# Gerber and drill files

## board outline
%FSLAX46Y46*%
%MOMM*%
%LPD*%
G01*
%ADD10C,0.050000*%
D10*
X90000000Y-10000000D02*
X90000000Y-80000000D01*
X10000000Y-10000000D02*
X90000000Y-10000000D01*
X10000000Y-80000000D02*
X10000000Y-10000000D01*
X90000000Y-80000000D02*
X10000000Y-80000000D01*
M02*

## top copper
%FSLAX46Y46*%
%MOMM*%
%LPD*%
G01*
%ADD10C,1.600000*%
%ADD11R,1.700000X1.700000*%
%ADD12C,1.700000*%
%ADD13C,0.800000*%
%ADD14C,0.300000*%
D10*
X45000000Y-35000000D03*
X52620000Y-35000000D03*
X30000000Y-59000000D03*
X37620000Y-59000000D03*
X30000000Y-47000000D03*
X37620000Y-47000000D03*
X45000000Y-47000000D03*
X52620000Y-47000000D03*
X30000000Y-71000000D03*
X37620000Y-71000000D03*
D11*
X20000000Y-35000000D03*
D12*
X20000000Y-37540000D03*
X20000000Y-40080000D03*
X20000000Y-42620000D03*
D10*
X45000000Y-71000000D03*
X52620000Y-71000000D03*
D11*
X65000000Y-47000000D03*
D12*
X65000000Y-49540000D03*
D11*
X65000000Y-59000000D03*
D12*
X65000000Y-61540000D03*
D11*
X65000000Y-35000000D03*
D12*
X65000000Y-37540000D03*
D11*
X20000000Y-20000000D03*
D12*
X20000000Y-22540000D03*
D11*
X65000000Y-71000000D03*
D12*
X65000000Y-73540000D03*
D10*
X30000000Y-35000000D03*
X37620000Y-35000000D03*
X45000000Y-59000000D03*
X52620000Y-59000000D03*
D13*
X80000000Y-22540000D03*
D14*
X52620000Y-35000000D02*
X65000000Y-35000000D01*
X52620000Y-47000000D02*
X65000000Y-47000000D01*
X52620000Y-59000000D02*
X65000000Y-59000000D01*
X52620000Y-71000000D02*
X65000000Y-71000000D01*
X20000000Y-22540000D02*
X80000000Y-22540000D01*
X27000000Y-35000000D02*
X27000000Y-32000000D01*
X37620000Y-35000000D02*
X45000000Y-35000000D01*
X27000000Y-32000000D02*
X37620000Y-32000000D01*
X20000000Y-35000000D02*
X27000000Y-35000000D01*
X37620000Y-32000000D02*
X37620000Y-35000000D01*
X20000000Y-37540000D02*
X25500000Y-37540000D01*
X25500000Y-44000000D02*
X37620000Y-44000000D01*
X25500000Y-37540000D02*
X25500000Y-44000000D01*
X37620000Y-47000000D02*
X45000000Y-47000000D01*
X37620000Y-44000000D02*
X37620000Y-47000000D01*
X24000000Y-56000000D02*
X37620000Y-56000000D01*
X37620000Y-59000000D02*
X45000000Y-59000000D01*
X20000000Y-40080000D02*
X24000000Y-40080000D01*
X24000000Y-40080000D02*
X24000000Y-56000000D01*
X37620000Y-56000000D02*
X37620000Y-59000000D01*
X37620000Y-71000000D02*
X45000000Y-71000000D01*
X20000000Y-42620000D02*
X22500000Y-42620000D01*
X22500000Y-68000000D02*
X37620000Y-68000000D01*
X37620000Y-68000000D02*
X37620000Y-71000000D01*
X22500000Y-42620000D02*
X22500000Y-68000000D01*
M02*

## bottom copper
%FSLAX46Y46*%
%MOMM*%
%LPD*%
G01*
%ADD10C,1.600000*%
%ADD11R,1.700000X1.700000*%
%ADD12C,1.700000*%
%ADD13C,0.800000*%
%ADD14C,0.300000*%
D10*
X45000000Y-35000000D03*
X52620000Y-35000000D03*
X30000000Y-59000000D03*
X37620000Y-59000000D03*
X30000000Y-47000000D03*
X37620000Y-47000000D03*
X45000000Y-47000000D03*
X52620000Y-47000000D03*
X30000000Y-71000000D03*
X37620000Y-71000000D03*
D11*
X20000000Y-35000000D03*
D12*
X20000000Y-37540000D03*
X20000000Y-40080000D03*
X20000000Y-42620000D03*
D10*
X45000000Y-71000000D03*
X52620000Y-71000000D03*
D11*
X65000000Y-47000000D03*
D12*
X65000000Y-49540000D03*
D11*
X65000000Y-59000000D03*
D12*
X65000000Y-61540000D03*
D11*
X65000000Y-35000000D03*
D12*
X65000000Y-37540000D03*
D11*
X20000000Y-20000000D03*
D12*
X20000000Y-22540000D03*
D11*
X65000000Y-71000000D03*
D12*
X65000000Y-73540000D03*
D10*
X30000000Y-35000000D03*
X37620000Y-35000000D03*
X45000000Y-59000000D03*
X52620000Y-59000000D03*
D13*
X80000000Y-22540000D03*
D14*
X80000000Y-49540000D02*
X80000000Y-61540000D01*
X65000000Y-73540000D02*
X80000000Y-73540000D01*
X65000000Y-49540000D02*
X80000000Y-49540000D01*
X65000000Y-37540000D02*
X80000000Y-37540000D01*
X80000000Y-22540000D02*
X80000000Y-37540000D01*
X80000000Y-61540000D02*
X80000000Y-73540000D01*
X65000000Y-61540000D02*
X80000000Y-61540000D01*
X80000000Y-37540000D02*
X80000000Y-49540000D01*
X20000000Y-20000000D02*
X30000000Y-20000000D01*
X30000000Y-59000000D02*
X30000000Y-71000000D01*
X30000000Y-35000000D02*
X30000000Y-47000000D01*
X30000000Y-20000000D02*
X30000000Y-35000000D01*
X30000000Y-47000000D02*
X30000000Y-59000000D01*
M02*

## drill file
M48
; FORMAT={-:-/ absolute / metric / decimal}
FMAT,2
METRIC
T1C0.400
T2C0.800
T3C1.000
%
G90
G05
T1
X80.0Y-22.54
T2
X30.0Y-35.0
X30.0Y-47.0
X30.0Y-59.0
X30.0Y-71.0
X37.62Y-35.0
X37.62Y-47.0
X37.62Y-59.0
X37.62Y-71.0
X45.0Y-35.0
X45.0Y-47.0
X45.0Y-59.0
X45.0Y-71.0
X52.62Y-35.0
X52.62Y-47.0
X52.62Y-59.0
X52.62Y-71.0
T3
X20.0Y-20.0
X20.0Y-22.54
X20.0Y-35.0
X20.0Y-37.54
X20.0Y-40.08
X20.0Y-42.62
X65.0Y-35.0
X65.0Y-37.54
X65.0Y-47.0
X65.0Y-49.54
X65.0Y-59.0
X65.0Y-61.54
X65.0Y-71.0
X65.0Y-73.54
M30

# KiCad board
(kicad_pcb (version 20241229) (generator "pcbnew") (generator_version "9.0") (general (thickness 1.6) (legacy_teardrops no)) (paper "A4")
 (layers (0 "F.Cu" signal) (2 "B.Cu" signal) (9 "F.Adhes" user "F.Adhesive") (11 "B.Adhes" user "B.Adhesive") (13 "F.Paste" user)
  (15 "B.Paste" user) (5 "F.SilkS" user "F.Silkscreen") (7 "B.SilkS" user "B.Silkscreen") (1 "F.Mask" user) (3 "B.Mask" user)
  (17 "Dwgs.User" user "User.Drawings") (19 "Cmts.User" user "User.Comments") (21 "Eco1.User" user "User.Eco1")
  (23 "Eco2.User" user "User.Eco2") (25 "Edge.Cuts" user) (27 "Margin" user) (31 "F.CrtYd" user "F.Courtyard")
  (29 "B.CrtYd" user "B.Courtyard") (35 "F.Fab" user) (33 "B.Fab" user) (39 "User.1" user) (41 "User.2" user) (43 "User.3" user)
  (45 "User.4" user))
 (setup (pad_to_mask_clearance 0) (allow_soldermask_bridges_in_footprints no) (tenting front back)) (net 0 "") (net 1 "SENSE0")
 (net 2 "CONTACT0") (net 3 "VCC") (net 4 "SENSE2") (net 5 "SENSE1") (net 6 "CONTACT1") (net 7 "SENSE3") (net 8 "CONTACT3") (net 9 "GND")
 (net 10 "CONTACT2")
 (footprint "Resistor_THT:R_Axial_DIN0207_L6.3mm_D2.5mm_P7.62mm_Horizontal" (layer "F.Cu") (at 45 35)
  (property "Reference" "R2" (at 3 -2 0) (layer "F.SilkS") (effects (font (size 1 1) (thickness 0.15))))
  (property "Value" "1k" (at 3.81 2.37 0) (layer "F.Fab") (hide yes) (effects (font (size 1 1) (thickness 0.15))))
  (pad "1" thru_hole circle (at 0 0) (size 1.6 1.6) (drill 0.8) (layers "*.Cu" "*.Mask") (remove_unused_layers no) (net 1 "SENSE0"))
  (pad "2" thru_hole circle (at 7.62 0) (size 1.6 1.6) (drill 0.8) (layers "*.Cu" "*.Mask") (remove_unused_layers no) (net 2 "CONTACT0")))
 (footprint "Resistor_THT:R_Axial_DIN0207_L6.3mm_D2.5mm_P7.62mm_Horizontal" (layer "F.Cu") (at 30 59)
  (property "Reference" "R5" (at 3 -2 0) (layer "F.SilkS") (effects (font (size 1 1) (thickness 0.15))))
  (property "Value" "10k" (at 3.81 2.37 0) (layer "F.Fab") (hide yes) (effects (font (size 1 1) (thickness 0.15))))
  (pad "1" thru_hole circle (at 0 0) (size 1.6 1.6) (drill 0.8) (layers "*.Cu" "*.Mask") (remove_unused_layers no) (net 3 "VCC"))
  (pad "2" thru_hole circle (at 7.62 0) (size 1.6 1.6) (drill 0.8) (layers "*.Cu" "*.Mask") (remove_unused_layers no) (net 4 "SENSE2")))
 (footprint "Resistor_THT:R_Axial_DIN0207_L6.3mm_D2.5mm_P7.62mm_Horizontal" (layer "F.Cu") (at 30 47)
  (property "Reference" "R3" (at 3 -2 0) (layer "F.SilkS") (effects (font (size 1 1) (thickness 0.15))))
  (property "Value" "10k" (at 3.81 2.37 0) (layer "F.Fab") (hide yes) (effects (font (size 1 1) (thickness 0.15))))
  (pad "1" thru_hole circle (at 0 0) (size 1.6 1.6) (drill 0.8) (layers "*.Cu" "*.Mask") (remove_unused_layers no) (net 3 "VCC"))
  (pad "2" thru_hole circle (at 7.62 0) (size 1.6 1.6) (drill 0.8) (layers "*.Cu" "*.Mask") (remove_unused_layers no) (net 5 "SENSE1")))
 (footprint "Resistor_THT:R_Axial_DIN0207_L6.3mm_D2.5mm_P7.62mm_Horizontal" (layer "F.Cu") (at 45 47)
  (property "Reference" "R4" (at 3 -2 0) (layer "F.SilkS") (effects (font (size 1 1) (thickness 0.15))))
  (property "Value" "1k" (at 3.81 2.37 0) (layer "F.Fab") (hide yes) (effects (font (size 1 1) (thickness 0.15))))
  (pad "1" thru_hole circle (at 0 0) (size 1.6 1.6) (drill 0.8) (layers "*.Cu" "*.Mask") (remove_unused_layers no) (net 5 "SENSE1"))
  (pad "2" thru_hole circle (at 7.62 0) (size 1.6 1.6) (drill 0.8) (layers "*.Cu" "*.Mask") (remove_unused_layers no) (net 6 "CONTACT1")))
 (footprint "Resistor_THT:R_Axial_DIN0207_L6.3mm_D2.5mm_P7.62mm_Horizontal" (layer "F.Cu") (at 30 71)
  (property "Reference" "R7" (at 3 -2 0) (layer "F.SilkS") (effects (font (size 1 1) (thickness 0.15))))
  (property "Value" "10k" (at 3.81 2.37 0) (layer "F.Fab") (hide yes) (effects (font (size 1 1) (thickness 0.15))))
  (pad "1" thru_hole circle (at 0 0) (size 1.6 1.6) (drill 0.8) (layers "*.Cu" "*.Mask") (remove_unused_layers no) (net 3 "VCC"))
  (pad "2" thru_hole circle (at 7.62 0) (size 1.6 1.6) (drill 0.8) (layers "*.Cu" "*.Mask") (remove_unused_layers no) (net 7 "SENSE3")))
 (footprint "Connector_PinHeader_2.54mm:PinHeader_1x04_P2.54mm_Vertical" (layer "F.Cu") (at 20 35)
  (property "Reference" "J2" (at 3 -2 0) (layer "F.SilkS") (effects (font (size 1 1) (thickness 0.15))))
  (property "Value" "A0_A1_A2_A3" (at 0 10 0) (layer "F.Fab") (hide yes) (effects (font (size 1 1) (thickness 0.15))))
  (pad "1" thru_hole rect (at 0 0) (size 1.7 1.7) (drill 1) (layers "*.Cu" "*.Mask") (remove_unused_layers no) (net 1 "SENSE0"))
  (pad "2" thru_hole circle (at 0 2.54) (size 1.7 1.7) (drill 1) (layers "*.Cu" "*.Mask") (remove_unused_layers no) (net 5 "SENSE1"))
  (pad "3" thru_hole circle (at 0 5.08) (size 1.7 1.7) (drill 1) (layers "*.Cu" "*.Mask") (remove_unused_layers no) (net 4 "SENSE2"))
  (pad "4" thru_hole circle (at 0 7.62) (size 1.7 1.7) (drill 1) (layers "*.Cu" "*.Mask") (remove_unused_layers no) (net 7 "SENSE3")))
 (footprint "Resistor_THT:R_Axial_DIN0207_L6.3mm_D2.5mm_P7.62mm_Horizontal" (layer "F.Cu") (at 45 71)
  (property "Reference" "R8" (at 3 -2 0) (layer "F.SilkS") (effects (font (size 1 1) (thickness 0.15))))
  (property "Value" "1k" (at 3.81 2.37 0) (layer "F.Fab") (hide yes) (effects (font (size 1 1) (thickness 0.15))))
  (pad "1" thru_hole circle (at 0 0) (size 1.6 1.6) (drill 0.8) (layers "*.Cu" "*.Mask") (remove_unused_layers no) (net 7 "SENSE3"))
  (pad "2" thru_hole circle (at 7.62 0) (size 1.6 1.6) (drill 0.8) (layers "*.Cu" "*.Mask") (remove_unused_layers no) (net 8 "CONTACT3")))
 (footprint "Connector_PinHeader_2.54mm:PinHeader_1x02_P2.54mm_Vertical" (layer "F.Cu") (at 65 47)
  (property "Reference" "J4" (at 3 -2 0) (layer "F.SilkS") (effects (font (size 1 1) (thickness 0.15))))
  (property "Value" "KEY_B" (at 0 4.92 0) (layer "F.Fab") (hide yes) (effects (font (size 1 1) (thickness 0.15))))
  (pad "1" thru_hole rect (at 0 0) (size 1.7 1.7) (drill 1) (layers "*.Cu" "*.Mask") (remove_unused_layers no) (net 6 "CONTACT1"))
  (pad "2" thru_hole circle (at 0 2.54) (size 1.7 1.7) (drill 1) (layers "*.Cu" "*.Mask") (remove_unused_layers no) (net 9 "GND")))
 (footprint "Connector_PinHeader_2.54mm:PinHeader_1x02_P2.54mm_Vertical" (layer "F.Cu") (at 65 59)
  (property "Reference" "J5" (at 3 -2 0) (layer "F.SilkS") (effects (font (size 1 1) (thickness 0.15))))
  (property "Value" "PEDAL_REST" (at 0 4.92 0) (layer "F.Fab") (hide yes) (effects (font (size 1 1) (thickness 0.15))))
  (pad "1" thru_hole rect (at 0 0) (size 1.7 1.7) (drill 1) (layers "*.Cu" "*.Mask") (remove_unused_layers no) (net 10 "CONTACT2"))
  (pad "2" thru_hole circle (at 0 2.54) (size 1.7 1.7) (drill 1) (layers "*.Cu" "*.Mask") (remove_unused_layers no) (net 9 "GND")))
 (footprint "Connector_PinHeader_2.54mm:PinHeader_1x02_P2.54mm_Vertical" (layer "F.Cu") (at 65 35)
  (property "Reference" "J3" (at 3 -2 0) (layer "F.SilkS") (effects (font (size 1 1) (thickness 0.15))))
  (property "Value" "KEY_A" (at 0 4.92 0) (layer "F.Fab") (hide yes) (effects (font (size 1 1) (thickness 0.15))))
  (pad "1" thru_hole rect (at 0 0) (size 1.7 1.7) (drill 1) (layers "*.Cu" "*.Mask") (remove_unused_layers no) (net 2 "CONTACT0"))
  (pad "2" thru_hole circle (at 0 2.54) (size 1.7 1.7) (drill 1) (layers "*.Cu" "*.Mask") (remove_unused_layers no) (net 9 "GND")))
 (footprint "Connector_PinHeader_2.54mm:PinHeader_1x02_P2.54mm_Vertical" (layer "F.Cu") (at 20 20)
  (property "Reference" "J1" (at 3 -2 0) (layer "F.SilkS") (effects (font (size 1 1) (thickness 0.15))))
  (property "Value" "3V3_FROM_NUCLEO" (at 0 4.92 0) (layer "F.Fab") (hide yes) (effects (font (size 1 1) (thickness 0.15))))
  (pad "1" thru_hole rect (at 0 0) (size 1.7 1.7) (drill 1) (layers "*.Cu" "*.Mask") (remove_unused_layers no) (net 3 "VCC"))
  (pad "2" thru_hole circle (at 0 2.54) (size 1.7 1.7) (drill 1) (layers "*.Cu" "*.Mask") (remove_unused_layers no) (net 9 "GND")))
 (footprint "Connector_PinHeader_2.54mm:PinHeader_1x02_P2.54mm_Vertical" (layer "F.Cu") (at 65 71)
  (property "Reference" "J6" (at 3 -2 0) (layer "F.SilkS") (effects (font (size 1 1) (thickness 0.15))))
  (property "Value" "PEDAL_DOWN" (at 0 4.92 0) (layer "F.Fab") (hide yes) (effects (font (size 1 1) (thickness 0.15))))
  (pad "1" thru_hole rect (at 0 0) (size 1.7 1.7) (drill 1) (layers "*.Cu" "*.Mask") (remove_unused_layers no) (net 8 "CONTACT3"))
  (pad "2" thru_hole circle (at 0 2.54) (size 1.7 1.7) (drill 1) (layers "*.Cu" "*.Mask") (remove_unused_layers no) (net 9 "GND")))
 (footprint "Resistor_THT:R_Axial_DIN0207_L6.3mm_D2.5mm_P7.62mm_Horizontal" (layer "F.Cu") (at 30 35)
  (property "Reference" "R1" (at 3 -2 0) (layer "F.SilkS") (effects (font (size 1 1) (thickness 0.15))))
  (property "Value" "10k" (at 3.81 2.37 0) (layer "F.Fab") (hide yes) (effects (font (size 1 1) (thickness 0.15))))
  (pad "1" thru_hole circle (at 0 0) (size 1.6 1.6) (drill 0.8) (layers "*.Cu" "*.Mask") (remove_unused_layers no) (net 3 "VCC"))
  (pad "2" thru_hole circle (at 7.62 0) (size 1.6 1.6) (drill 0.8) (layers "*.Cu" "*.Mask") (remove_unused_layers no) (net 1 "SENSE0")))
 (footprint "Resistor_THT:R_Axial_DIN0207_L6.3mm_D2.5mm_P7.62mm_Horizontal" (layer "F.Cu") (at 45 59)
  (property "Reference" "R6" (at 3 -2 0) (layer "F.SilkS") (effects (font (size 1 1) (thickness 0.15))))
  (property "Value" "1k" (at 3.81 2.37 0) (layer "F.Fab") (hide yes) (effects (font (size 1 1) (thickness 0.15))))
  (pad "1" thru_hole circle (at 0 0) (size 1.6 1.6) (drill 0.8) (layers "*.Cu" "*.Mask") (remove_unused_layers no) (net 4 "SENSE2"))
  (pad "2" thru_hole circle (at 7.62 0) (size 1.6 1.6) (drill 0.8) (layers "*.Cu" "*.Mask") (remove_unused_layers no) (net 10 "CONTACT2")))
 (gr_line (start 90 10) (end 90 80) (stroke (width 0.05) (type default)) (layer "Edge.Cuts"))
 (gr_line (start 10 10) (end 90 10) (stroke (width 0.05) (type default)) (layer "Edge.Cuts"))
 (gr_line (start 10 80) (end 10 10) (stroke (width 0.05) (type default)) (layer "Edge.Cuts"))
 (gr_line (start 90 80) (end 10 80) (stroke (width 0.05) (type default)) (layer "Edge.Cuts"))
 (segment (start 52.62 35) (end 65 35) (width 0.3) (layer "F.Cu") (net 2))
 (segment (start 52.62 47) (end 65 47) (width 0.3) (layer "F.Cu") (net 6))
 (segment (start 52.62 59) (end 65 59) (width 0.3) (layer "F.Cu") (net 10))
 (segment (start 52.62 71) (end 65 71) (width 0.3) (layer "F.Cu") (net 8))
 (segment (start 20 22.54) (end 80 22.54) (width 0.3) (layer "F.Cu") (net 9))
 (via (at 80 22.54) (size 0.8) (drill 0.4) (layers "F.Cu" "B.Cu") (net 9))
 (segment (start 80 49.54) (end 80 61.54) (width 0.3) (layer "B.Cu") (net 9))
 (segment (start 65 73.54) (end 80 73.54) (width 0.3) (layer "B.Cu") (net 9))
 (segment (start 65 49.54) (end 80 49.54) (width 0.3) (layer "B.Cu") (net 9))
 (segment (start 65 37.54) (end 80 37.54) (width 0.3) (layer "B.Cu") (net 9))
 (segment (start 80 22.54) (end 80 37.54) (width 0.3) (layer "B.Cu") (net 9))
 (segment (start 80 61.54) (end 80 73.54) (width 0.3) (layer "B.Cu") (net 9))
 (segment (start 65 61.54) (end 80 61.54) (width 0.3) (layer "B.Cu") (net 9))
 (segment (start 80 37.54) (end 80 49.54) (width 0.3) (layer "B.Cu") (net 9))
 (segment (start 27 35) (end 27 32) (width 0.3) (layer "F.Cu") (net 1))
 (segment (start 37.62 35) (end 45 35) (width 0.3) (layer "F.Cu") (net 1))
 (segment (start 27 32) (end 37.62 32) (width 0.3) (layer "F.Cu") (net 1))
 (segment (start 20 35) (end 27 35) (width 0.3) (layer "F.Cu") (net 1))
 (segment (start 37.62 32) (end 37.62 35) (width 0.3) (layer "F.Cu") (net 1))
 (segment (start 20 37.54) (end 25.5 37.54) (width 0.3) (layer "F.Cu") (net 5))
 (segment (start 25.5 44) (end 37.62 44) (width 0.3) (layer "F.Cu") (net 5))
 (segment (start 25.5 37.54) (end 25.5 44) (width 0.3) (layer "F.Cu") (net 5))
 (segment (start 37.62 47) (end 45 47) (width 0.3) (layer "F.Cu") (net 5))
 (segment (start 37.62 44) (end 37.62 47) (width 0.3) (layer "F.Cu") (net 5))
 (segment (start 24 56) (end 37.62 56) (width 0.3) (layer "F.Cu") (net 4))
 (segment (start 37.62 59) (end 45 59) (width 0.3) (layer "F.Cu") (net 4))
 (segment (start 20 40.08) (end 24 40.08) (width 0.3) (layer "F.Cu") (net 4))
 (segment (start 24 40.08) (end 24 56) (width 0.3) (layer "F.Cu") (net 4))
 (segment (start 37.62 56) (end 37.62 59) (width 0.3) (layer "F.Cu") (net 4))
 (segment (start 37.62 71) (end 45 71) (width 0.3) (layer "F.Cu") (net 7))
 (segment (start 20 42.62) (end 22.5 42.62) (width 0.3) (layer "F.Cu") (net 7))
 (segment (start 22.5 68) (end 37.62 68) (width 0.3) (layer "F.Cu") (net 7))
 (segment (start 37.62 68) (end 37.62 71) (width 0.3) (layer "F.Cu") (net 7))
 (segment (start 22.5 42.62) (end 22.5 68) (width 0.3) (layer "F.Cu") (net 7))
 (segment (start 20 20) (end 30 20) (width 0.3) (layer "B.Cu") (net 3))
 (segment (start 30 59) (end 30 71) (width 0.3) (layer "B.Cu") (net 3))
 (segment (start 30 35) (end 30 47) (width 0.3) (layer "B.Cu") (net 3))
 (segment (start 30 20) (end 30 35) (width 0.3) (layer "B.Cu") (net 3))
 (segment (start 30 47) (end 30 59) (width 0.3) (layer "B.Cu") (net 3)))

